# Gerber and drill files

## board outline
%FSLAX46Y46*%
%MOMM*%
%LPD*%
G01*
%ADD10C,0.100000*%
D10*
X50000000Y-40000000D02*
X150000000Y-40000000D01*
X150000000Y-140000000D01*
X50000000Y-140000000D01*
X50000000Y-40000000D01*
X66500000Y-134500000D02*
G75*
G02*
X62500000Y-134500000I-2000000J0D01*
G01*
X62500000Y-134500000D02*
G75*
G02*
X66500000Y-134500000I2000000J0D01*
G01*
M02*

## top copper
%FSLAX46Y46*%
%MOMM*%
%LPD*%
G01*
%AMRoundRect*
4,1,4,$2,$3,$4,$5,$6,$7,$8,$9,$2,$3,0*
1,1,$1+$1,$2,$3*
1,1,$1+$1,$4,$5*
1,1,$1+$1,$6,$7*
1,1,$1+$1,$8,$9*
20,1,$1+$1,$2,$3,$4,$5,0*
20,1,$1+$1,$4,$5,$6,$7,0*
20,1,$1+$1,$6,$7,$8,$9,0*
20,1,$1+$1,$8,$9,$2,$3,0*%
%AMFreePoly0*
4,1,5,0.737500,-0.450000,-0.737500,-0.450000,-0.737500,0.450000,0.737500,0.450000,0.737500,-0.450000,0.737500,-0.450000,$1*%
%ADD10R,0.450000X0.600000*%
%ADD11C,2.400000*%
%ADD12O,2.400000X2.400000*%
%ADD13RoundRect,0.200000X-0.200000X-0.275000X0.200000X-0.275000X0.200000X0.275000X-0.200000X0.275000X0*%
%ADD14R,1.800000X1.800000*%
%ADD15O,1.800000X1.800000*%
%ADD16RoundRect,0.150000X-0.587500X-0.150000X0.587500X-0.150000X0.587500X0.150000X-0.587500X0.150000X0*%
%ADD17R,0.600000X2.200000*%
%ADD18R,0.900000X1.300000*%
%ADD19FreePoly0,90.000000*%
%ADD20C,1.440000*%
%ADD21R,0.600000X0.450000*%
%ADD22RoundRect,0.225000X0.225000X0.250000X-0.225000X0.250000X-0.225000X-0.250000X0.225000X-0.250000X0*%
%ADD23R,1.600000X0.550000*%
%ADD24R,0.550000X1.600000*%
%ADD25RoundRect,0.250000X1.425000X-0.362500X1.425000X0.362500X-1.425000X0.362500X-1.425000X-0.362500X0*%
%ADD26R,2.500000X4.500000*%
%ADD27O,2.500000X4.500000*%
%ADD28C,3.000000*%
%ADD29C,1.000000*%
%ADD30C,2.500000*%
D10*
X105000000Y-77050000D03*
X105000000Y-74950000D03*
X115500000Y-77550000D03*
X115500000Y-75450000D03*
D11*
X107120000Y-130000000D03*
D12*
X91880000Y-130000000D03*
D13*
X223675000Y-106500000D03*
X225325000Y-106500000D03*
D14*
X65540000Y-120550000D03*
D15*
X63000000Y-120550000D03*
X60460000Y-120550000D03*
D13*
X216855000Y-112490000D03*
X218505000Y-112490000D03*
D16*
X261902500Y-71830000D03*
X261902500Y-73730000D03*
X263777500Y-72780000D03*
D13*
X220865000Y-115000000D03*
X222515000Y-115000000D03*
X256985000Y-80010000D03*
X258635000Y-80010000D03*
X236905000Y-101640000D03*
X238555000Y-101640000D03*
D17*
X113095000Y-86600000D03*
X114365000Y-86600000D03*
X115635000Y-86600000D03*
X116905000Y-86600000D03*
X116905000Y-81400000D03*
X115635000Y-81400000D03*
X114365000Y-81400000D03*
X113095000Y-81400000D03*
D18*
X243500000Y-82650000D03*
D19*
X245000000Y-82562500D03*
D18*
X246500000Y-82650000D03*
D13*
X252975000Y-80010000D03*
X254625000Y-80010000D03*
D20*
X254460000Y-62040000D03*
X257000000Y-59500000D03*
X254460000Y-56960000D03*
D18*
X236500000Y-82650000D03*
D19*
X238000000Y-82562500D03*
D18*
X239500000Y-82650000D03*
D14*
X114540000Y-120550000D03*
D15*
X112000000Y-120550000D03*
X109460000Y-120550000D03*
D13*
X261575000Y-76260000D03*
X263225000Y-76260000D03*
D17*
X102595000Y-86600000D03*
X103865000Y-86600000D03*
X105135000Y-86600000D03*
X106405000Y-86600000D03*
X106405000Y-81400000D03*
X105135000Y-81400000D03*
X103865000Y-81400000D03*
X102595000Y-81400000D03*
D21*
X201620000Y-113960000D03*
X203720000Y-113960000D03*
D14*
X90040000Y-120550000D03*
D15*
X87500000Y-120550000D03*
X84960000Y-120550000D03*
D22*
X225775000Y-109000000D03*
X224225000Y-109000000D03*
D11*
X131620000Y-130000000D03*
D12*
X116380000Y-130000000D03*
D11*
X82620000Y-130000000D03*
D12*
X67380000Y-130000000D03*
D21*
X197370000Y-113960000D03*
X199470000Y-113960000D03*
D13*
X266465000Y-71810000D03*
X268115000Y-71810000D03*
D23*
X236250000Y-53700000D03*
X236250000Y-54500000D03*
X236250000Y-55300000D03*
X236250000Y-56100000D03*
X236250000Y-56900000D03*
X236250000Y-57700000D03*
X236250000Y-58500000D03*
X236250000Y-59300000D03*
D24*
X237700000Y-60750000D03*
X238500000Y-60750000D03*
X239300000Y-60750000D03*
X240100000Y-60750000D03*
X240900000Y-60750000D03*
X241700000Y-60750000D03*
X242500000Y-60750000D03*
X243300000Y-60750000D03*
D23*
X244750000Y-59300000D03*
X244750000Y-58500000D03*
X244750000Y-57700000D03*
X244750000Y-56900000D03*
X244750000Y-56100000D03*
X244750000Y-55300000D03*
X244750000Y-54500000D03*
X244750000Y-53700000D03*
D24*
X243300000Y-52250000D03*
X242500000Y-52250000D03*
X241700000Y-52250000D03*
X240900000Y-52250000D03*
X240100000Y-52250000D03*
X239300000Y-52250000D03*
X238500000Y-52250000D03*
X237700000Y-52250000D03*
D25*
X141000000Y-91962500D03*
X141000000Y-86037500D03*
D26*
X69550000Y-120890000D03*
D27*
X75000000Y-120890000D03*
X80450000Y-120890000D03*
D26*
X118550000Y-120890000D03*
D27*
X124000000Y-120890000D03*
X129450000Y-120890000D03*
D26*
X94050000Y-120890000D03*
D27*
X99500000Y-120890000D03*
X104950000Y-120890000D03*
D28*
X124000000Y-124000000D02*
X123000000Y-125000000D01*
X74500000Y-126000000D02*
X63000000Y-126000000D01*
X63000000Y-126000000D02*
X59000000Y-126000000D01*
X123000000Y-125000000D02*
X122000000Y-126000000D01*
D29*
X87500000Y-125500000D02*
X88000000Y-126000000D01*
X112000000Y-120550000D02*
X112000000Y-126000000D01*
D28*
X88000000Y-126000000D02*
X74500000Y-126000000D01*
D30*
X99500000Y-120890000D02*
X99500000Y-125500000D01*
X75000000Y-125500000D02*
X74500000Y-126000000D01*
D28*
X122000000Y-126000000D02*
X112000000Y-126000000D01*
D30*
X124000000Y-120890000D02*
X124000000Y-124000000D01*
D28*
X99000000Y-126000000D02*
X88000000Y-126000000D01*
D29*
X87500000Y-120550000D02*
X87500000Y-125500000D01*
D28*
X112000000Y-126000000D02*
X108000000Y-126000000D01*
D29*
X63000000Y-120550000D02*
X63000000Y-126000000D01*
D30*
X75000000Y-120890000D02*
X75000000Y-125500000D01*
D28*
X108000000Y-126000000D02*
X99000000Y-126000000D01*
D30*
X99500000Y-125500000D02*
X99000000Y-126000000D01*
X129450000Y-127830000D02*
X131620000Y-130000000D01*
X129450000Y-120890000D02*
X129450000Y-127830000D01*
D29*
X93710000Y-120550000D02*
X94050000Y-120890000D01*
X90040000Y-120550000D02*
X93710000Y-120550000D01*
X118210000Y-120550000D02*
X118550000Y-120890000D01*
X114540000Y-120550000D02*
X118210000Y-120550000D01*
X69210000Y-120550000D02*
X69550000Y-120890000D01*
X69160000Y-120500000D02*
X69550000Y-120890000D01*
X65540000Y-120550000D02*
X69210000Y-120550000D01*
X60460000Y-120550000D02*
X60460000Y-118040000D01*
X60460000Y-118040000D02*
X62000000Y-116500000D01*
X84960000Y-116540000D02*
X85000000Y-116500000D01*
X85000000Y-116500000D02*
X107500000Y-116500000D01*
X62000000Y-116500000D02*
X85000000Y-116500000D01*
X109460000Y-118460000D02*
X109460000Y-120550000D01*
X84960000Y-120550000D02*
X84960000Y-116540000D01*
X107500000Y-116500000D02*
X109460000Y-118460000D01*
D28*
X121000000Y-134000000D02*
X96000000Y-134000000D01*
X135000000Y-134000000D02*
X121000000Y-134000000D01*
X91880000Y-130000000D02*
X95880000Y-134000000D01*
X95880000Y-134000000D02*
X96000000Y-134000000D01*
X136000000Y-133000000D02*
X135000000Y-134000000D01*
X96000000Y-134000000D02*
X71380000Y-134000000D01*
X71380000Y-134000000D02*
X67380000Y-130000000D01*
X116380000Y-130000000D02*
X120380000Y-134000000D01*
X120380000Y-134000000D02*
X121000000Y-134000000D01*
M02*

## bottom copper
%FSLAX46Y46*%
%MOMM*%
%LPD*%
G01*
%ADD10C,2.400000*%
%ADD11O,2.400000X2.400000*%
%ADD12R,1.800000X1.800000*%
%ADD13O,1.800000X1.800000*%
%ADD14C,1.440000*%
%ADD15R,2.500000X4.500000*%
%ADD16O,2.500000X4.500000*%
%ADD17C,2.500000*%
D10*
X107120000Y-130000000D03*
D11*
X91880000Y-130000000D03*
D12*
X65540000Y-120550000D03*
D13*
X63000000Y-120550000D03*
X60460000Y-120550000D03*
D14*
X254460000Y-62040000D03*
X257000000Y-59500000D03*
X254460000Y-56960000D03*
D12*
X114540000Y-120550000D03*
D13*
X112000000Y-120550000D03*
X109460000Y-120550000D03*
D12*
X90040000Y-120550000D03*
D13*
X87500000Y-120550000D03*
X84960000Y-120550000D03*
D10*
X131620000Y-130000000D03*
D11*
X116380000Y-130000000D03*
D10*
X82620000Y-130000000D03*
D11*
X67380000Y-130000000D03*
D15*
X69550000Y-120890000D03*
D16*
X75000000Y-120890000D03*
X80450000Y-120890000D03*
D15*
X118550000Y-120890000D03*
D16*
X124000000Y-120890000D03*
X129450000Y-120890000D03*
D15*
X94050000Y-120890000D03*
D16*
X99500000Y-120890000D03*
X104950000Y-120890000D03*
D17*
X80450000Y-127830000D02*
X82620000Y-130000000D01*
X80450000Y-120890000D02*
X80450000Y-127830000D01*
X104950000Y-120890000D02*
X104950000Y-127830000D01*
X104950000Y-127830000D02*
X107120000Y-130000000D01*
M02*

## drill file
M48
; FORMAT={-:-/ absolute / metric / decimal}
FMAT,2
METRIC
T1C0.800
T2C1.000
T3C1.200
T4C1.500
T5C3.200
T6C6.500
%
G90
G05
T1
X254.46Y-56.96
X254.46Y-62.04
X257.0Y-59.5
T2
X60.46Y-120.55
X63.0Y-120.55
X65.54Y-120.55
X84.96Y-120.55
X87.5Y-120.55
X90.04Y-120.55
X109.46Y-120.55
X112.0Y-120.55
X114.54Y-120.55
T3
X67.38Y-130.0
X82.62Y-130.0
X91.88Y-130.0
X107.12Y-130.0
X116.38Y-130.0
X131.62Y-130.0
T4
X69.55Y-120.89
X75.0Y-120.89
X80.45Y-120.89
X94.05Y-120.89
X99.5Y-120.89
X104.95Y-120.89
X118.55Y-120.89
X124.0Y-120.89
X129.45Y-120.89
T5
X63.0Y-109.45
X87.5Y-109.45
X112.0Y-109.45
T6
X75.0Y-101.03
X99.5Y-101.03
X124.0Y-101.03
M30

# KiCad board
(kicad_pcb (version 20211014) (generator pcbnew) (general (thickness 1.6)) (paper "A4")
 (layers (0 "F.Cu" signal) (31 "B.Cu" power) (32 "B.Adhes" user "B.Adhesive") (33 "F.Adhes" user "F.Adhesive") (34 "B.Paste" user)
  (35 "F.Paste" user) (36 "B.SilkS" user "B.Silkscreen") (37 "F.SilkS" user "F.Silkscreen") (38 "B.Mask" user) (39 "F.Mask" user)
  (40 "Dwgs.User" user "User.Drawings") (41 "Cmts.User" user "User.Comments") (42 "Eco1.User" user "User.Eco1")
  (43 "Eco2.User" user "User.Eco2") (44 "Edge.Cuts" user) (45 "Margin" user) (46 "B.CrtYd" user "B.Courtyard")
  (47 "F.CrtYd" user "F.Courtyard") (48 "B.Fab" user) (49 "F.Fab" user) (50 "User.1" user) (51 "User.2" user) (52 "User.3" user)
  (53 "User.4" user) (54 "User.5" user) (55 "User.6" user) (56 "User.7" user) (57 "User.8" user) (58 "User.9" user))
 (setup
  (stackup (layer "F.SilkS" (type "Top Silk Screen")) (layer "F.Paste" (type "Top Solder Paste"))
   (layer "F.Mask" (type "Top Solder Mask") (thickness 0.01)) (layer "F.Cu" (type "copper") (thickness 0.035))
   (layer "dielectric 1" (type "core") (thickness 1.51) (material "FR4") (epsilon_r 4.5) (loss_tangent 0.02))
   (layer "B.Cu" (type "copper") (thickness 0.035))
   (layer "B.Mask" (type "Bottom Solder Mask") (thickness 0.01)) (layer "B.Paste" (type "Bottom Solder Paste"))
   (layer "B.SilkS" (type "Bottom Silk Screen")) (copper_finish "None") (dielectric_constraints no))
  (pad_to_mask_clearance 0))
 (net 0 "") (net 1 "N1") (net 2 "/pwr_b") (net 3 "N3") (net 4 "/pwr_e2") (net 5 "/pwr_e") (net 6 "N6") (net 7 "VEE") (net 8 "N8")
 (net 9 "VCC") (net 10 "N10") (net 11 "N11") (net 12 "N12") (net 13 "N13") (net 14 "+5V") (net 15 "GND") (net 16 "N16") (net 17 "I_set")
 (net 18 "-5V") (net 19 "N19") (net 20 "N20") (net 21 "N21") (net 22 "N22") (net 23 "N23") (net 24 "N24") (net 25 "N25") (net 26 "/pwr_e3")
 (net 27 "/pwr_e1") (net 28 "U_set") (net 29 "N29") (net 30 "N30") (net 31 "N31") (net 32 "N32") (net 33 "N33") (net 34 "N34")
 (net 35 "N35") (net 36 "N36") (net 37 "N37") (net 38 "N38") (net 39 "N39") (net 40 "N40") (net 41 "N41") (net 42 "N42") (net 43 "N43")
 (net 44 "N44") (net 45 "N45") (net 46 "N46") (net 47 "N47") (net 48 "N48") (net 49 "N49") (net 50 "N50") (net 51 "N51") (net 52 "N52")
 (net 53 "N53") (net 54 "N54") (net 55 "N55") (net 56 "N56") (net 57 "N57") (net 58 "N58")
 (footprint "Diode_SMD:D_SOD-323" (layer "F.Cu") (at 105 76 90)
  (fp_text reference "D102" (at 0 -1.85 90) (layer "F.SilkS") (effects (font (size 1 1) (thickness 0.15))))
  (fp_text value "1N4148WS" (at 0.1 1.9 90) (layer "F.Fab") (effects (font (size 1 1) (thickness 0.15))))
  (pad "1" smd rect (at -1.05 0 90) (size 0.6 0.45) (layers "F.Cu" "F.Paste" "F.Mask") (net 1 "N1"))
  (pad "2" smd rect (at 1.05 0 90) (size 0.6 0.45) (layers "F.Cu" "F.Paste" "F.Mask") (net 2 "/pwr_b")))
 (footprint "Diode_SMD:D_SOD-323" (layer "F.Cu") (at 115.5 76.5 90)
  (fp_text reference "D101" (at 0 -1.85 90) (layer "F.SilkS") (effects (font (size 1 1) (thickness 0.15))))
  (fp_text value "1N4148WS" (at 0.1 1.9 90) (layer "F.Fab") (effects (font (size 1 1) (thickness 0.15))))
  (pad "1" smd rect (at -1.05 0 90) (size 0.6 0.45) (layers "F.Cu" "F.Paste" "F.Mask") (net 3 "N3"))
  (pad "2" smd rect (at 1.05 0 90) (size 0.6 0.45) (layers "F.Cu" "F.Paste" "F.Mask") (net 2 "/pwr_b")))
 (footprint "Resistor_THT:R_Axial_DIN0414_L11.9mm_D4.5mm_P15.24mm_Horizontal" (layer "F.Cu") (at 107.12 130 180)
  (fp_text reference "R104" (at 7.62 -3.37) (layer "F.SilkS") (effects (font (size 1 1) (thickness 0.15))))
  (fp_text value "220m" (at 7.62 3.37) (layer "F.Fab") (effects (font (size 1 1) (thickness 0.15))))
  (pad "1" thru_hole circle (at 0 0 180) (size 2.4 2.4) (drill 1.2) (layers *.Cu *.Mask) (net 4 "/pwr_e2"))
  (pad "2" thru_hole oval (at 15.24 0 180) (size 2.4 2.4) (drill 1.2) (layers *.Cu *.Mask) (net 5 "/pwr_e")))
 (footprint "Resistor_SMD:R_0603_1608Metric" (layer "F.Cu") (at 224.5 106.5)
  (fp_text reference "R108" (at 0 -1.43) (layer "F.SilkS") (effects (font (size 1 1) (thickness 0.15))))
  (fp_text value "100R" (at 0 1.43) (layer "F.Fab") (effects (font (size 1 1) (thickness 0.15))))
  (pad "1" smd roundrect (at -0.825 0) (size 0.8 0.95) (layers "F.Cu" "F.Paste" "F.Mask") (roundrect_rratio 0.25) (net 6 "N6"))
  (pad "2" smd roundrect (at 0.825 0) (size 0.8 0.95) (layers "F.Cu" "F.Paste" "F.Mask") (roundrect_rratio 0.25) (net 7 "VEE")))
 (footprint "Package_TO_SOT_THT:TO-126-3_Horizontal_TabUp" (layer "F.Cu") (at 65.54 120.55 180)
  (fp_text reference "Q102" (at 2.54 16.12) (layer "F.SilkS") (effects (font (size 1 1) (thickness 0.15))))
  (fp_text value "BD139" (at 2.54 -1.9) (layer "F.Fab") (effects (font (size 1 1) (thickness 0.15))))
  (pad "" np_thru_hole oval (at 2.54 11.1 180) (size 3.2 3.2) (drill 3.2) (layers *.Cu *.Mask))
  (pad "1" thru_hole rect (at 0 0 180) (size 1.8 1.8) (drill 1) (layers *.Cu *.Mask) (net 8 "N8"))
  (pad "2" thru_hole oval (at 2.54 0 180) (size 1.8 1.8) (drill 1) (layers *.Cu *.Mask) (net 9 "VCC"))
  (pad "3" thru_hole oval (at 5.08 0 180) (size 1.8 1.8) (drill 1) (layers *.Cu *.Mask) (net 2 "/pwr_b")))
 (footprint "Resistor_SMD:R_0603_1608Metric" (layer "F.Cu") (at 217.68 112.49)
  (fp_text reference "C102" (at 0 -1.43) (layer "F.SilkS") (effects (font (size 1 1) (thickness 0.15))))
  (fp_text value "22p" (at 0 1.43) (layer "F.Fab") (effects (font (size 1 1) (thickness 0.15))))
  (pad "1" smd roundrect (at -0.825 0) (size 0.8 0.95) (layers "F.Cu" "F.Paste" "F.Mask") (roundrect_rratio 0.25) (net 3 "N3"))
  (pad "2" smd roundrect (at 0.825 0) (size 0.8 0.95) (layers "F.Cu" "F.Paste" "F.Mask") (roundrect_rratio 0.25) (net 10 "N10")))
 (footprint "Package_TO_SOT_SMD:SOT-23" (layer "F.Cu") (at 262.84 72.78)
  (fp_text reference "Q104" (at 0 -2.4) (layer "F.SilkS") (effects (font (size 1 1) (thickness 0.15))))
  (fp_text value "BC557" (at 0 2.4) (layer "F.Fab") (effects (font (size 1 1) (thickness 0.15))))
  (pad "1" smd roundrect (at -0.9375 -0.95) (size 1.475 0.6) (layers "F.Cu" "F.Paste" "F.Mask") (roundrect_rratio 0.25) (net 2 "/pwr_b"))
  (pad "2" smd roundrect (at -0.9375 0.95) (size 1.475 0.6) (layers "F.Cu" "F.Paste" "F.Mask") (roundrect_rratio 0.25) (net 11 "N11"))
  (pad "3" smd roundrect (at 0.9375 0) (size 1.475 0.6) (layers "F.Cu" "F.Paste" "F.Mask") (roundrect_rratio 0.25) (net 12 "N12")))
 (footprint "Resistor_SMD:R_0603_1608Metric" (layer "F.Cu") (at 221.69 115)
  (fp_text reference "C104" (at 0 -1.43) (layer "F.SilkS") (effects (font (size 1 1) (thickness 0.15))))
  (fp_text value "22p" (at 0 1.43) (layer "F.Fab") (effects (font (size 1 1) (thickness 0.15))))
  (pad "1" smd roundrect (at -0.825 0) (size 0.8 0.95) (layers "F.Cu" "F.Paste" "F.Mask") (roundrect_rratio 0.25) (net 1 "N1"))
  (pad "2" smd roundrect (at 0.825 0) (size 0.8 0.95) (layers "F.Cu" "F.Paste" "F.Mask") (roundrect_rratio 0.25) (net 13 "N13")))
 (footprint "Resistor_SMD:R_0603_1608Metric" (layer "F.Cu") (at 257.81 80.01)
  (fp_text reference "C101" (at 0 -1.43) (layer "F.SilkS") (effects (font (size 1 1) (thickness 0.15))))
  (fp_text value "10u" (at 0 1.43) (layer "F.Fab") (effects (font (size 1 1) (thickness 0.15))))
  (pad "1" smd roundrect (at -0.825 0) (size 0.8 0.95) (layers "F.Cu" "F.Paste" "F.Mask") (roundrect_rratio 0.25) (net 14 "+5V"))
  (pad "2" smd roundrect (at 0.825 0) (size 0.8 0.95) (layers "F.Cu" "F.Paste" "F.Mask") (roundrect_rratio 0.25) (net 11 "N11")))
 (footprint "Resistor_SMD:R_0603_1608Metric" (layer "F.Cu") (at 237.73 101.64)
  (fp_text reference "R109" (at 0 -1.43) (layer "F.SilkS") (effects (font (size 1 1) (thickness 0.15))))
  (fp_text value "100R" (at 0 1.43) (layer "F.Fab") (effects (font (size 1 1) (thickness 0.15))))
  (pad "1" smd roundrect (at -0.825 0) (size 0.8 0.95) (layers "F.Cu" "F.Paste" "F.Mask") (roundrect_rratio 0.25) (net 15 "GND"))
  (pad "2" smd roundrect (at 0.825 0) (size 0.8 0.95) (layers "F.Cu" "F.Paste" "F.Mask") (roundrect_rratio 0.25) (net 13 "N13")))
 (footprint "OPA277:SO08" (layer "F.Cu") (at 115 84)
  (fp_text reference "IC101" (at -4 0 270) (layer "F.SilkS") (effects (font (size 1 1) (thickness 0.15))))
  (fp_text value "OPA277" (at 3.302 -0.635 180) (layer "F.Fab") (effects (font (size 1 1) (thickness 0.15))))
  (pad "1" smd rect locked (at -1.905 2.6) (size 0.6 2.2) (layers "F.Cu" "F.Paste" "F.Mask") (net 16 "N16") (solder_mask_margin 0.102))
  (pad "2" smd rect locked (at -0.635 2.6) (size 0.6 2.2) (layers "F.Cu" "F.Paste" "F.Mask") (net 10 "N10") (solder_mask_margin 0.102))
  (pad "3" smd rect locked (at 0.635 2.6) (size 0.6 2.2) (layers "F.Cu" "F.Paste" "F.Mask") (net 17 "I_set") (solder_mask_margin 0.102))
  (pad "4" smd rect locked (at 1.905 2.6) (size 0.6 2.2) (layers "F.Cu" "F.Paste" "F.Mask") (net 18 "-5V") (solder_mask_margin 0.102))
  (pad "5" smd rect locked (at 1.905 -2.6) (size 0.6 2.2) (layers "F.Cu" "F.Paste" "F.Mask") (solder_mask_margin 0.102))
  (pad "6" smd rect locked (at 0.635 -2.6) (size 0.6 2.2) (layers "F.Cu" "F.Paste" "F.Mask") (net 3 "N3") (solder_mask_margin 0.102))
  (pad "7" smd rect locked (at -0.635 -2.6) (size 0.6 2.2) (layers "F.Cu" "F.Paste" "F.Mask") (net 14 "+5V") (solder_mask_margin 0.102))
  (pad "8" smd rect locked (at -1.905 -2.6) (size 0.6 2.2) (layers "F.Cu" "F.Paste" "F.Mask") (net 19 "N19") (solder_mask_margin 0.102)))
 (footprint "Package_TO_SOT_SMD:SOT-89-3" (layer "F.Cu") (at 245 81 90)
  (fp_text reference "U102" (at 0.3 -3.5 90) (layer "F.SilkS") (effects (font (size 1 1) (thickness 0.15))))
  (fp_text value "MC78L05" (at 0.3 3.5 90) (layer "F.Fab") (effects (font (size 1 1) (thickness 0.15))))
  (pad "1" smd rect (at -1.65 -1.5 90) (size 1.3 0.9) (layers "F.Cu" "F.Paste" "F.Mask") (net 14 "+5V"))
  (pad "2" smd custom (at -1.5625 0 90) (size 1.475 0.9) (layers "F.Cu" "F.Paste" "F.Mask") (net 15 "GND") (zone_connect 2)
   (options (clearance outline) (anchor rect)) (primitives))
  (pad "3" smd rect (at -1.65 1.5 90) (size 1.3 0.9) (layers "F.Cu" "F.Paste" "F.Mask") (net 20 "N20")))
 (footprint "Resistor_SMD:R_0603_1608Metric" (layer "F.Cu") (at 253.8 80.01)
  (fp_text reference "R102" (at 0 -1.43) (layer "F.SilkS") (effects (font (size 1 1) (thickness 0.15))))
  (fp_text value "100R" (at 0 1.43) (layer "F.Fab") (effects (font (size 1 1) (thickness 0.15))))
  (pad "1" smd roundrect (at -0.825 0) (size 0.8 0.95) (layers "F.Cu" "F.Paste" "F.Mask") (roundrect_rratio 0.25) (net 12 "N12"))
  (pad "2" smd roundrect (at 0.825 0) (size 0.8 0.95) (layers "F.Cu" "F.Paste" "F.Mask") (roundrect_rratio 0.25) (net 14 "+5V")))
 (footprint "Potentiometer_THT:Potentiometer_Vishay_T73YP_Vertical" (layer "F.Cu") (at 254.46 62.04)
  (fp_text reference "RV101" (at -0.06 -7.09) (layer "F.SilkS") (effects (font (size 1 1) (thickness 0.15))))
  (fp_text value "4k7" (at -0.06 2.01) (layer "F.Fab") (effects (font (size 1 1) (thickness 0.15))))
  (pad "1" thru_hole circle (at 0 0) (size 1.44 1.44) (drill 0.8) (layers *.Cu *.Mask) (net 14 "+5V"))
  (pad "2" thru_hole circle (at 2.54 -2.54) (size 1.44 1.44) (drill 0.8) (layers *.Cu *.Mask) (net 11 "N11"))
  (pad "3" thru_hole circle (at 0 -5.08) (size 1.44 1.44) (drill 0.8) (layers *.Cu *.Mask) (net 15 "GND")))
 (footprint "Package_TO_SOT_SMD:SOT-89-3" (layer "F.Cu") (at 238 81 90)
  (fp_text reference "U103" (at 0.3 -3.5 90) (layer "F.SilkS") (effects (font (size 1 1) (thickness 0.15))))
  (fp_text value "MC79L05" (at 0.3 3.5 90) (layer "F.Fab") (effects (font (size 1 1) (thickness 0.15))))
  (pad "1" smd rect (at -1.65 -1.5 90) (size 1.3 0.9) (layers "F.Cu" "F.Paste" "F.Mask") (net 15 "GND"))
  (pad "2" smd custom (at -1.5625 0 90) (size 1.475 0.9) (layers "F.Cu" "F.Paste" "F.Mask") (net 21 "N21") (zone_connect 2)
   (options (clearance outline) (anchor rect)) (primitives))
  (pad "3" smd rect (at -1.65 1.5 90) (size 1.3 0.9) (layers "F.Cu" "F.Paste" "F.Mask") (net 18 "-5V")))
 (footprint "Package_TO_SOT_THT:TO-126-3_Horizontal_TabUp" (layer "F.Cu") (at 114.54 120.55 180)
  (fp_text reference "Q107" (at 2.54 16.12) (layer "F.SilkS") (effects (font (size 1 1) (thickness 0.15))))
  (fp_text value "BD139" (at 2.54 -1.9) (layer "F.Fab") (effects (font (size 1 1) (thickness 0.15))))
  (pad "" np_thru_hole oval (at 2.54 11.1 180) (size 3.2 3.2) (drill 3.2) (layers *.Cu *.Mask))
  (pad "1" thru_hole rect (at 0 0 180) (size 1.8 1.8) (drill 1) (layers *.Cu *.Mask) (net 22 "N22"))
  (pad "2" thru_hole oval (at 2.54 0 180) (size 1.8 1.8) (drill 1) (layers *.Cu *.Mask) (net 9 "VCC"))
  (pad "3" thru_hole oval (at 5.08 0 180) (size 1.8 1.8) (drill 1) (layers *.Cu *.Mask) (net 2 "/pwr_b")))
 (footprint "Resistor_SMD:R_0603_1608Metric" (layer "F.Cu") (at 262.4 76.26)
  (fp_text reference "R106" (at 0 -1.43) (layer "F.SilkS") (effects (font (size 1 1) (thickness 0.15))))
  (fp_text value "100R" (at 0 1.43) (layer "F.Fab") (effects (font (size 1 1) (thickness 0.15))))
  (pad "1" smd roundrect (at -0.825 0) (size 0.8 0.95) (layers "F.Cu" "F.Paste" "F.Mask") (roundrect_rratio 0.25) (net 5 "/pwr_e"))
  (pad "2" smd roundrect (at 0.825 0) (size 0.8 0.95) (layers "F.Cu" "F.Paste" "F.Mask") (roundrect_rratio 0.25) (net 10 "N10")))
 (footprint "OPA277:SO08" (layer "F.Cu") (at 104.5 84)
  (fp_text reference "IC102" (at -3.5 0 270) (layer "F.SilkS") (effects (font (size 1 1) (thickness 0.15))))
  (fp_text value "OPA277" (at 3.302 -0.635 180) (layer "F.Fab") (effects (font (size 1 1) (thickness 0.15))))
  (pad "1" smd rect locked (at -1.905 2.6) (size 0.6 2.2) (layers "F.Cu" "F.Paste" "F.Mask") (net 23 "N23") (solder_mask_margin 0.102))
  (pad "2" smd rect locked (at -0.635 2.6) (size 0.6 2.2) (layers "F.Cu" "F.Paste" "F.Mask") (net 13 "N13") (solder_mask_margin 0.102))
  (pad "3" smd rect locked (at 0.635 2.6) (size 0.6 2.2) (layers "F.Cu" "F.Paste" "F.Mask") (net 6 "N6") (solder_mask_margin 0.102))
  (pad "4" smd rect locked (at 1.905 2.6) (size 0.6 2.2) (layers "F.Cu" "F.Paste" "F.Mask") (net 18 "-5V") (solder_mask_margin 0.102))
  (pad "5" smd rect locked (at 1.905 -2.6) (size 0.6 2.2) (layers "F.Cu" "F.Paste" "F.Mask") (solder_mask_margin 0.102))
  (pad "6" smd rect locked (at 0.635 -2.6) (size 0.6 2.2) (layers "F.Cu" "F.Paste" "F.Mask") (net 1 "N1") (solder_mask_margin 0.102))
  (pad "7" smd rect locked (at -0.635 -2.6) (size 0.6 2.2) (layers "F.Cu" "F.Paste" "F.Mask") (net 14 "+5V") (solder_mask_margin 0.102))
  (pad "8" smd rect locked (at -1.905 -2.6) (size 0.6 2.2) (layers "F.Cu" "F.Paste" "F.Mask") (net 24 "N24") (solder_mask_margin 0.102)))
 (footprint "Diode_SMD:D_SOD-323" (layer "F.Cu") (at 202.67 113.96)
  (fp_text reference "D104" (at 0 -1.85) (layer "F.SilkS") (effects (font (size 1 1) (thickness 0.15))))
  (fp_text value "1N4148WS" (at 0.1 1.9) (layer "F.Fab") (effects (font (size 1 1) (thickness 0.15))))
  (pad "1" smd rect (at -1.05 0) (size 0.6 0.45) (layers "F.Cu" "F.Paste" "F.Mask") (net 6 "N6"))
  (pad "2" smd rect (at 1.05 0) (size 0.6 0.45) (layers "F.Cu" "F.Paste" "F.Mask") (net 15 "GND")))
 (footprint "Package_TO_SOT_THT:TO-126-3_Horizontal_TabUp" (layer "F.Cu") (at 90.04 120.55 180)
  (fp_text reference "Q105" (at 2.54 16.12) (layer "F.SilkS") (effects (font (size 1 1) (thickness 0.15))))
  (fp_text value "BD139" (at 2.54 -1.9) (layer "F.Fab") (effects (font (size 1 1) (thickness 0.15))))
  (pad "" np_thru_hole oval (at 2.54 11.1 180) (size 3.2 3.2) (drill 3.2) (layers *.Cu *.Mask))
  (pad "1" thru_hole rect (at 0 0 180) (size 1.8 1.8) (drill 1) (layers *.Cu *.Mask) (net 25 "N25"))
  (pad "2" thru_hole oval (at 2.54 0 180) (size 1.8 1.8) (drill 1) (layers *.Cu *.Mask) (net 9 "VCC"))
  (pad "3" thru_hole oval (at 5.08 0 180) (size 1.8 1.8) (drill 1) (layers *.Cu *.Mask) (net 2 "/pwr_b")))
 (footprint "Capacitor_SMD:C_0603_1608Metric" (layer "F.Cu") (at 225 109 180)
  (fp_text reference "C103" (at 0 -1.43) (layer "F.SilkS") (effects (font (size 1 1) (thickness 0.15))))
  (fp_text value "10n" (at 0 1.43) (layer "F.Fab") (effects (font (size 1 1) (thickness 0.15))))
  (pad "1" smd roundrect (at -0.775 0 180) (size 0.9 0.95) (layers "F.Cu" "F.Paste" "F.Mask") (roundrect_rratio 0.25) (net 7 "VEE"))
  (pad "2" smd roundrect (at 0.775 0 180) (size 0.9 0.95) (layers "F.Cu" "F.Paste" "F.Mask") (roundrect_rratio 0.25) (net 6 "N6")))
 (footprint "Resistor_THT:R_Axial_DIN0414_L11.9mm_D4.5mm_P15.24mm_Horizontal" (layer "F.Cu") (at 131.62 130 180)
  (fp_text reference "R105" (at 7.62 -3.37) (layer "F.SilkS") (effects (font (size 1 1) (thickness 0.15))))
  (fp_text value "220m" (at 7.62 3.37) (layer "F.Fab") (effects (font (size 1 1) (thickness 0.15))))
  (pad "1" thru_hole circle (at 0 0 180) (size 2.4 2.4) (drill 1.2) (layers *.Cu *.Mask) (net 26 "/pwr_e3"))
  (pad "2" thru_hole oval (at 15.24 0 180) (size 2.4 2.4) (drill 1.2) (layers *.Cu *.Mask) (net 5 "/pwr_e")))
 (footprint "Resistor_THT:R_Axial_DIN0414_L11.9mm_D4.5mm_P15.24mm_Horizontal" (layer "F.Cu") (at 82.62 130 180)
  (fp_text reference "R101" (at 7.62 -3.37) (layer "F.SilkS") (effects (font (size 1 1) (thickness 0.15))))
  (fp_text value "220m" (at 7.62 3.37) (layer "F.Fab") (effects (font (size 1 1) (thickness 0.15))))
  (pad "1" thru_hole circle (at 0 0 180) (size 2.4 2.4) (drill 1.2) (layers *.Cu *.Mask) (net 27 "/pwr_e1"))
  (pad "2" thru_hole oval (at 15.24 0 180) (size 2.4 2.4) (drill 1.2) (layers *.Cu *.Mask) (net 5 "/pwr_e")))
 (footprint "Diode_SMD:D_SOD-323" (layer "F.Cu") (at 198.42 113.96)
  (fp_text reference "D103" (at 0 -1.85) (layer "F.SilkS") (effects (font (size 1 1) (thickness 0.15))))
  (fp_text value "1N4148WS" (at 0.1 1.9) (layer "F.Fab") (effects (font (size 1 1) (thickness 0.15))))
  (pad "1" smd rect (at -1.05 0) (size 0.6 0.45) (layers "F.Cu" "F.Paste" "F.Mask") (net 15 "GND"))
  (pad "2" smd rect (at 1.05 0) (size 0.6 0.45) (layers "F.Cu" "F.Paste" "F.Mask") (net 6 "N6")))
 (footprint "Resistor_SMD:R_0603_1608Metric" (layer "F.Cu") (at 267.29 71.81)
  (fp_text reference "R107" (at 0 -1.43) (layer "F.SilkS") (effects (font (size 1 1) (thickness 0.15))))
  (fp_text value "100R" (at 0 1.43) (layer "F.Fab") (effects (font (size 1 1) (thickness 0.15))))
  (pad "1" smd roundrect (at -0.825 0) (size 0.8 0.95) (layers "F.Cu" "F.Paste" "F.Mask") (roundrect_rratio 0.25) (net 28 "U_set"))
  (pad "2" smd roundrect (at 0.825 0) (size 0.8 0.95) (layers "F.Cu" "F.Paste" "F.Mask") (roundrect_rratio 0.25) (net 6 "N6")))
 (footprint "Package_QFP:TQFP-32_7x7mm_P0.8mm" (layer "F.Cu") (at 240.5 56.5)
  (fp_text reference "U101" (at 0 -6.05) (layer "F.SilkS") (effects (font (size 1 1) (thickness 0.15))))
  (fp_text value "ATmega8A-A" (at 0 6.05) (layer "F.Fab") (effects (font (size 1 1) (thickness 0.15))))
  (pad "1" smd rect (at -4.25 -2.8) (size 1.6 0.55) (layers "F.Cu" "F.Paste" "F.Mask") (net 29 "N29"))
  (pad "2" smd rect (at -4.25 -2) (size 1.6 0.55) (layers "F.Cu" "F.Paste" "F.Mask") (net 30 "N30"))
  (pad "3" smd rect (at -4.25 -1.2) (size 1.6 0.55) (layers "F.Cu" "F.Paste" "F.Mask") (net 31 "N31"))
  (pad "4" smd rect (at -4.25 -0.4) (size 1.6 0.55) (layers "F.Cu" "F.Paste" "F.Mask") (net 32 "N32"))
  (pad "5" smd rect (at -4.25 0.4) (size 1.6 0.55) (layers "F.Cu" "F.Paste" "F.Mask") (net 31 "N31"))
  (pad "6" smd rect (at -4.25 1.2) (size 1.6 0.55) (layers "F.Cu" "F.Paste" "F.Mask") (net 32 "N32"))
  (pad "7" smd rect (at -4.25 2) (size 1.6 0.55) (layers "F.Cu" "F.Paste" "F.Mask") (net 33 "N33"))
  (pad "8" smd rect (at -4.25 2.8) (size 1.6 0.55) (layers "F.Cu" "F.Paste" "F.Mask") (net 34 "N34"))
  (pad "9" smd rect (at -2.8 4.25 90) (size 1.6 0.55) (layers "F.Cu" "F.Paste" "F.Mask") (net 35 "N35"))
  (pad "10" smd rect (at -2 4.25 90) (size 1.6 0.55) (layers "F.Cu" "F.Paste" "F.Mask") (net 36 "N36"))
  (pad "11" smd rect (at -1.2 4.25 90) (size 1.6 0.55) (layers "F.Cu" "F.Paste" "F.Mask") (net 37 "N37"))
  (pad "12" smd rect (at -0.4 4.25 90) (size 1.6 0.55) (layers "F.Cu" "F.Paste" "F.Mask") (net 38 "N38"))
  (pad "13" smd rect (at 0.4 4.25 90) (size 1.6 0.55) (layers "F.Cu" "F.Paste" "F.Mask") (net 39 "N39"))
  (pad "14" smd rect (at 1.2 4.25 90) (size 1.6 0.55) (layers "F.Cu" "F.Paste" "F.Mask") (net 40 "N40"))
  (pad "15" smd rect (at 2 4.25 90) (size 1.6 0.55) (layers "F.Cu" "F.Paste" "F.Mask") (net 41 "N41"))
  (pad "16" smd rect (at 2.8 4.25 90) (size 1.6 0.55) (layers "F.Cu" "F.Paste" "F.Mask") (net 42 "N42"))
  (pad "17" smd rect (at 4.25 2.8) (size 1.6 0.55) (layers "F.Cu" "F.Paste" "F.Mask") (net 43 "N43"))
  (pad "18" smd rect (at 4.25 2) (size 1.6 0.55) (layers "F.Cu" "F.Paste" "F.Mask") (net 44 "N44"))
  (pad "19" smd rect (at 4.25 1.2) (size 1.6 0.55) (layers "F.Cu" "F.Paste" "F.Mask") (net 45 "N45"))
  (pad "20" smd rect (at 4.25 0.4) (size 1.6 0.55) (layers "F.Cu" "F.Paste" "F.Mask") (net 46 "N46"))
  (pad "21" smd rect (at 4.25 -0.4) (size 1.6 0.55) (layers "F.Cu" "F.Paste" "F.Mask") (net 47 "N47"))
  (pad "22" smd rect (at 4.25 -1.2) (size 1.6 0.55) (layers "F.Cu" "F.Paste" "F.Mask") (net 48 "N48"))
  (pad "23" smd rect (at 4.25 -2) (size 1.6 0.55) (layers "F.Cu" "F.Paste" "F.Mask") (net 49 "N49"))
  (pad "24" smd rect (at 4.25 -2.8) (size 1.6 0.55) (layers "F.Cu" "F.Paste" "F.Mask") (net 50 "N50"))
  (pad "25" smd rect (at 2.8 -4.25 90) (size 1.6 0.55) (layers "F.Cu" "F.Paste" "F.Mask") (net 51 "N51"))
  (pad "26" smd rect (at 2 -4.25 90) (size 1.6 0.55) (layers "F.Cu" "F.Paste" "F.Mask") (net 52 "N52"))
  (pad "27" smd rect (at 1.2 -4.25 90) (size 1.6 0.55) (layers "F.Cu" "F.Paste" "F.Mask") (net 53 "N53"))
  (pad "28" smd rect (at 0.4 -4.25 90) (size 1.6 0.55) (layers "F.Cu" "F.Paste" "F.Mask") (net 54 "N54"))
  (pad "29" smd rect (at -0.4 -4.25 90) (size 1.6 0.55) (layers "F.Cu" "F.Paste" "F.Mask") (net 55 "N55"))
  (pad "30" smd rect (at -1.2 -4.25 90) (size 1.6 0.55) (layers "F.Cu" "F.Paste" "F.Mask") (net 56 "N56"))
  (pad "31" smd rect (at -2 -4.25 90) (size 1.6 0.55) (layers "F.Cu" "F.Paste" "F.Mask") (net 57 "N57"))
  (pad "32" smd rect (at -2.8 -4.25 90) (size 1.6 0.55) (layers "F.Cu" "F.Paste" "F.Mask") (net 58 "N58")))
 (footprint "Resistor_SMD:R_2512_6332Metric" (layer "F.Cu") (at 141 89 90)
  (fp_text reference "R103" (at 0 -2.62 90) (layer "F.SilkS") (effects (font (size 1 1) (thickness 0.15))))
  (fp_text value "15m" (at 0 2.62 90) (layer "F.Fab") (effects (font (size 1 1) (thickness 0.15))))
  (pad "1" smd roundrect (at -2.9625 0 90) (size 1.225 3.35) (layers "F.Cu" "F.Paste" "F.Mask") (roundrect_rratio 0.204082) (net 5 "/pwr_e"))
  (pad "2" smd roundrect (at 2.9625 0 90) (size 1.225 3.35) (layers "F.Cu" "F.Paste" "F.Mask") (roundrect_rratio 0.204082) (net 15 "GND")))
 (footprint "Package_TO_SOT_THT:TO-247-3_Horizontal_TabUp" (layer "B.Cu") (at 69.55 120.89)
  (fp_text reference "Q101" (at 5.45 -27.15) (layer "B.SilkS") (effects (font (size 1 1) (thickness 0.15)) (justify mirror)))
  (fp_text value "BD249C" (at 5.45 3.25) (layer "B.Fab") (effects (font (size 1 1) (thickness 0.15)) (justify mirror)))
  (pad "" np_thru_hole circle (at 5.45 -19.86) (size 6.5 6.5) (drill 6.5) (layers F&B.Cu *.Mask))
  (pad "1" thru_hole rect (at 0 0) (size 2.5 4.5) (drill 1.5) (layers *.Cu *.Mask) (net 8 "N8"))
  (pad "2" thru_hole oval (at 5.45 0) (size 2.5 4.5) (drill 1.5) (layers *.Cu *.Mask) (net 9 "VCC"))
  (pad "3" thru_hole oval (at 10.9 0) (size 2.5 4.5) (drill 1.5) (layers *.Cu *.Mask) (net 27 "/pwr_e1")))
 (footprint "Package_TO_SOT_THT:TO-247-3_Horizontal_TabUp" (layer "B.Cu") (at 118.55 120.89)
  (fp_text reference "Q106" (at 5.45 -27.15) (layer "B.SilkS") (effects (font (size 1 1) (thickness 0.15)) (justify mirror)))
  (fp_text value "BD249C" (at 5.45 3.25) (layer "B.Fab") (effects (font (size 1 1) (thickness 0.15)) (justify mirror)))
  (pad "" np_thru_hole circle (at 5.45 -19.86) (size 6.5 6.5) (drill 6.5) (layers F&B.Cu *.Mask))
  (pad "1" thru_hole rect (at 0 0) (size 2.5 4.5) (drill 1.5) (layers *.Cu *.Mask) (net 22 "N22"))
  (pad "2" thru_hole oval (at 5.45 0) (size 2.5 4.5) (drill 1.5) (layers *.Cu *.Mask) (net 9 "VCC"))
  (pad "3" thru_hole oval (at 10.9 0) (size 2.5 4.5) (drill 1.5) (layers *.Cu *.Mask) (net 26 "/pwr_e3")))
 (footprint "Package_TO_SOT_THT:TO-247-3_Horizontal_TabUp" (layer "B.Cu") (at 94.05 120.89)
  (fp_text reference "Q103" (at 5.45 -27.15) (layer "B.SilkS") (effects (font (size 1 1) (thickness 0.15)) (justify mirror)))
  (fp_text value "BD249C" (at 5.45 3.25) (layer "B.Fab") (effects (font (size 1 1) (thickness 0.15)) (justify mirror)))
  (pad "" np_thru_hole circle (at 5.45 -19.86) (size 6.5 6.5) (drill 6.5) (layers F&B.Cu *.Mask))
  (pad "1" thru_hole rect (at 0 0) (size 2.5 4.5) (drill 1.5) (layers *.Cu *.Mask) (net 25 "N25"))
  (pad "2" thru_hole oval (at 5.45 0) (size 2.5 4.5) (drill 1.5) (layers *.Cu *.Mask) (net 9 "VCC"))
  (pad "3" thru_hole oval (at 10.9 0) (size 2.5 4.5) (drill 1.5) (layers *.Cu *.Mask) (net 4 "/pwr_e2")))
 (gr_rect (start 50 40) (end 150 140) (layer "Edge.Cuts") (width 0.1) (fill none))
 (gr_circle (center 64.5 134.5) (end 64.5 132.5) (layer "Edge.Cuts") (width 0.1) (fill none))
 (segment (start 124 124) (end 123 125) (width 3) (layer "F.Cu") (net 9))
 (segment (start 74.5 126) (end 63 126) (width 3) (layer "F.Cu") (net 9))
 (segment (start 63 126) (end 59 126) (width 3) (layer "F.Cu") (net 9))
 (segment (start 123 125) (end 122 126) (width 3) (layer "F.Cu") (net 9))
 (segment (start 87.5 125.5) (end 88 126) (width 1) (layer "F.Cu") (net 9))
 (segment (start 112 120.55) (end 112 126) (width 1) (layer "F.Cu") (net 9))
 (segment (start 88 126) (end 74.5 126) (width 3) (layer "F.Cu") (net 9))
 (segment (start 99.5 120.89) (end 99.5 125.5) (width 2.5) (layer "F.Cu") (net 9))
 (segment (start 75 125.5) (end 74.5 126) (width 2.5) (layer "F.Cu") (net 9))
 (segment (start 122 126) (end 112 126) (width 3) (layer "F.Cu") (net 9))
 (segment (start 124 120.89) (end 124 124) (width 2.5) (layer "F.Cu") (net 9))
 (segment (start 99 126) (end 88 126) (width 3) (layer "F.Cu") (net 9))
 (segment (start 87.5 120.55) (end 87.5 125.5) (width 1) (layer "F.Cu") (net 9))
 (segment (start 112 126) (end 108 126) (width 3) (layer "F.Cu") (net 9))
 (segment (start 63 120.55) (end 63 126) (width 1) (layer "F.Cu") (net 9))
 (segment (start 75 120.89) (end 75 125.5) (width 2.5) (layer "F.Cu") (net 9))
 (segment (start 108 126) (end 99 126) (width 3) (layer "F.Cu") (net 9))
 (segment (start 99.5 125.5) (end 99 126) (width 2.5) (layer "F.Cu") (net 9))
 (segment (start 80.45 127.83) (end 82.62 130) (width 2.5) (layer "B.Cu") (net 27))
 (segment (start 80.45 120.89) (end 80.45 127.83) (width 2.5) (layer "B.Cu") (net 27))
 (segment (start 104.95 120.89) (end 104.95 127.83) (width 2.5) (layer "B.Cu") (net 4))
 (segment (start 104.95 127.83) (end 107.12 130) (width 2.5) (layer "B.Cu") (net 4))
 (segment (start 129.45 127.83) (end 131.62 130) (width 2.5) (layer "F.Cu") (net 26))
 (segment (start 129.45 120.89) (end 129.45 127.83) (width 2.5) (layer "F.Cu") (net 26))
 (segment (start 93.71 120.55) (end 94.05 120.89) (width 1) (layer "F.Cu") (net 25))
 (segment (start 90.04 120.55) (end 93.71 120.55) (width 1) (layer "F.Cu") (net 25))
 (segment (start 118.21 120.55) (end 118.55 120.89) (width 1) (layer "F.Cu") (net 22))
 (segment (start 114.54 120.55) (end 118.21 120.55) (width 1) (layer "F.Cu") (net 22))
 (segment (start 69.21 120.55) (end 69.55 120.89) (width 1) (layer "F.Cu") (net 8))
 (segment (start 69.16 120.5) (end 69.55 120.89) (width 1) (layer "F.Cu") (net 8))
 (segment (start 65.54 120.55) (end 69.21 120.55) (width 1) (layer "F.Cu") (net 8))
 (segment (start 60.46 120.55) (end 60.46 118.04) (width 1) (layer "F.Cu") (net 2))
 (segment (start 60.46 118.04) (end 62 116.5) (width 1) (layer "F.Cu") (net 2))
 (segment (start 84.96 116.54) (end 85 116.5) (width 1) (layer "F.Cu") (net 2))
 (segment (start 85 116.5) (end 107.5 116.5) (width 1) (layer "F.Cu") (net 2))
 (segment (start 62 116.5) (end 85 116.5) (width 1) (layer "F.Cu") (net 2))
 (segment (start 109.46 118.46) (end 109.46 120.55) (width 1) (layer "F.Cu") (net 2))
 (segment (start 84.96 120.55) (end 84.96 116.54) (width 1) (layer "F.Cu") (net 2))
 (segment (start 107.5 116.5) (end 109.46 118.46) (width 1) (layer "F.Cu") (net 2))
 (segment (start 121 134) (end 96 134) (width 3) (layer "F.Cu") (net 5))
 (segment (start 135 134) (end 121 134) (width 3) (layer "F.Cu") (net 5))
 (segment (start 91.88 130) (end 95.88 134) (width 3) (layer "F.Cu") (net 5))
 (segment (start 95.88 134) (end 96 134) (width 3) (layer "F.Cu") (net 5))
 (segment (start 136 133) (end 135 134) (width 3) (layer "F.Cu") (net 5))
 (segment (start 96 134) (end 71.38 134) (width 3) (layer "F.Cu") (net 5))
 (segment (start 71.38 134) (end 67.38 130) (width 3) (layer "F.Cu") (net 5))
 (segment (start 116.38 130) (end 120.38 134) (width 3) (layer "F.Cu") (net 5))
 (segment (start 120.38 134) (end 121 134) (width 3) (layer "F.Cu") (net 5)))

